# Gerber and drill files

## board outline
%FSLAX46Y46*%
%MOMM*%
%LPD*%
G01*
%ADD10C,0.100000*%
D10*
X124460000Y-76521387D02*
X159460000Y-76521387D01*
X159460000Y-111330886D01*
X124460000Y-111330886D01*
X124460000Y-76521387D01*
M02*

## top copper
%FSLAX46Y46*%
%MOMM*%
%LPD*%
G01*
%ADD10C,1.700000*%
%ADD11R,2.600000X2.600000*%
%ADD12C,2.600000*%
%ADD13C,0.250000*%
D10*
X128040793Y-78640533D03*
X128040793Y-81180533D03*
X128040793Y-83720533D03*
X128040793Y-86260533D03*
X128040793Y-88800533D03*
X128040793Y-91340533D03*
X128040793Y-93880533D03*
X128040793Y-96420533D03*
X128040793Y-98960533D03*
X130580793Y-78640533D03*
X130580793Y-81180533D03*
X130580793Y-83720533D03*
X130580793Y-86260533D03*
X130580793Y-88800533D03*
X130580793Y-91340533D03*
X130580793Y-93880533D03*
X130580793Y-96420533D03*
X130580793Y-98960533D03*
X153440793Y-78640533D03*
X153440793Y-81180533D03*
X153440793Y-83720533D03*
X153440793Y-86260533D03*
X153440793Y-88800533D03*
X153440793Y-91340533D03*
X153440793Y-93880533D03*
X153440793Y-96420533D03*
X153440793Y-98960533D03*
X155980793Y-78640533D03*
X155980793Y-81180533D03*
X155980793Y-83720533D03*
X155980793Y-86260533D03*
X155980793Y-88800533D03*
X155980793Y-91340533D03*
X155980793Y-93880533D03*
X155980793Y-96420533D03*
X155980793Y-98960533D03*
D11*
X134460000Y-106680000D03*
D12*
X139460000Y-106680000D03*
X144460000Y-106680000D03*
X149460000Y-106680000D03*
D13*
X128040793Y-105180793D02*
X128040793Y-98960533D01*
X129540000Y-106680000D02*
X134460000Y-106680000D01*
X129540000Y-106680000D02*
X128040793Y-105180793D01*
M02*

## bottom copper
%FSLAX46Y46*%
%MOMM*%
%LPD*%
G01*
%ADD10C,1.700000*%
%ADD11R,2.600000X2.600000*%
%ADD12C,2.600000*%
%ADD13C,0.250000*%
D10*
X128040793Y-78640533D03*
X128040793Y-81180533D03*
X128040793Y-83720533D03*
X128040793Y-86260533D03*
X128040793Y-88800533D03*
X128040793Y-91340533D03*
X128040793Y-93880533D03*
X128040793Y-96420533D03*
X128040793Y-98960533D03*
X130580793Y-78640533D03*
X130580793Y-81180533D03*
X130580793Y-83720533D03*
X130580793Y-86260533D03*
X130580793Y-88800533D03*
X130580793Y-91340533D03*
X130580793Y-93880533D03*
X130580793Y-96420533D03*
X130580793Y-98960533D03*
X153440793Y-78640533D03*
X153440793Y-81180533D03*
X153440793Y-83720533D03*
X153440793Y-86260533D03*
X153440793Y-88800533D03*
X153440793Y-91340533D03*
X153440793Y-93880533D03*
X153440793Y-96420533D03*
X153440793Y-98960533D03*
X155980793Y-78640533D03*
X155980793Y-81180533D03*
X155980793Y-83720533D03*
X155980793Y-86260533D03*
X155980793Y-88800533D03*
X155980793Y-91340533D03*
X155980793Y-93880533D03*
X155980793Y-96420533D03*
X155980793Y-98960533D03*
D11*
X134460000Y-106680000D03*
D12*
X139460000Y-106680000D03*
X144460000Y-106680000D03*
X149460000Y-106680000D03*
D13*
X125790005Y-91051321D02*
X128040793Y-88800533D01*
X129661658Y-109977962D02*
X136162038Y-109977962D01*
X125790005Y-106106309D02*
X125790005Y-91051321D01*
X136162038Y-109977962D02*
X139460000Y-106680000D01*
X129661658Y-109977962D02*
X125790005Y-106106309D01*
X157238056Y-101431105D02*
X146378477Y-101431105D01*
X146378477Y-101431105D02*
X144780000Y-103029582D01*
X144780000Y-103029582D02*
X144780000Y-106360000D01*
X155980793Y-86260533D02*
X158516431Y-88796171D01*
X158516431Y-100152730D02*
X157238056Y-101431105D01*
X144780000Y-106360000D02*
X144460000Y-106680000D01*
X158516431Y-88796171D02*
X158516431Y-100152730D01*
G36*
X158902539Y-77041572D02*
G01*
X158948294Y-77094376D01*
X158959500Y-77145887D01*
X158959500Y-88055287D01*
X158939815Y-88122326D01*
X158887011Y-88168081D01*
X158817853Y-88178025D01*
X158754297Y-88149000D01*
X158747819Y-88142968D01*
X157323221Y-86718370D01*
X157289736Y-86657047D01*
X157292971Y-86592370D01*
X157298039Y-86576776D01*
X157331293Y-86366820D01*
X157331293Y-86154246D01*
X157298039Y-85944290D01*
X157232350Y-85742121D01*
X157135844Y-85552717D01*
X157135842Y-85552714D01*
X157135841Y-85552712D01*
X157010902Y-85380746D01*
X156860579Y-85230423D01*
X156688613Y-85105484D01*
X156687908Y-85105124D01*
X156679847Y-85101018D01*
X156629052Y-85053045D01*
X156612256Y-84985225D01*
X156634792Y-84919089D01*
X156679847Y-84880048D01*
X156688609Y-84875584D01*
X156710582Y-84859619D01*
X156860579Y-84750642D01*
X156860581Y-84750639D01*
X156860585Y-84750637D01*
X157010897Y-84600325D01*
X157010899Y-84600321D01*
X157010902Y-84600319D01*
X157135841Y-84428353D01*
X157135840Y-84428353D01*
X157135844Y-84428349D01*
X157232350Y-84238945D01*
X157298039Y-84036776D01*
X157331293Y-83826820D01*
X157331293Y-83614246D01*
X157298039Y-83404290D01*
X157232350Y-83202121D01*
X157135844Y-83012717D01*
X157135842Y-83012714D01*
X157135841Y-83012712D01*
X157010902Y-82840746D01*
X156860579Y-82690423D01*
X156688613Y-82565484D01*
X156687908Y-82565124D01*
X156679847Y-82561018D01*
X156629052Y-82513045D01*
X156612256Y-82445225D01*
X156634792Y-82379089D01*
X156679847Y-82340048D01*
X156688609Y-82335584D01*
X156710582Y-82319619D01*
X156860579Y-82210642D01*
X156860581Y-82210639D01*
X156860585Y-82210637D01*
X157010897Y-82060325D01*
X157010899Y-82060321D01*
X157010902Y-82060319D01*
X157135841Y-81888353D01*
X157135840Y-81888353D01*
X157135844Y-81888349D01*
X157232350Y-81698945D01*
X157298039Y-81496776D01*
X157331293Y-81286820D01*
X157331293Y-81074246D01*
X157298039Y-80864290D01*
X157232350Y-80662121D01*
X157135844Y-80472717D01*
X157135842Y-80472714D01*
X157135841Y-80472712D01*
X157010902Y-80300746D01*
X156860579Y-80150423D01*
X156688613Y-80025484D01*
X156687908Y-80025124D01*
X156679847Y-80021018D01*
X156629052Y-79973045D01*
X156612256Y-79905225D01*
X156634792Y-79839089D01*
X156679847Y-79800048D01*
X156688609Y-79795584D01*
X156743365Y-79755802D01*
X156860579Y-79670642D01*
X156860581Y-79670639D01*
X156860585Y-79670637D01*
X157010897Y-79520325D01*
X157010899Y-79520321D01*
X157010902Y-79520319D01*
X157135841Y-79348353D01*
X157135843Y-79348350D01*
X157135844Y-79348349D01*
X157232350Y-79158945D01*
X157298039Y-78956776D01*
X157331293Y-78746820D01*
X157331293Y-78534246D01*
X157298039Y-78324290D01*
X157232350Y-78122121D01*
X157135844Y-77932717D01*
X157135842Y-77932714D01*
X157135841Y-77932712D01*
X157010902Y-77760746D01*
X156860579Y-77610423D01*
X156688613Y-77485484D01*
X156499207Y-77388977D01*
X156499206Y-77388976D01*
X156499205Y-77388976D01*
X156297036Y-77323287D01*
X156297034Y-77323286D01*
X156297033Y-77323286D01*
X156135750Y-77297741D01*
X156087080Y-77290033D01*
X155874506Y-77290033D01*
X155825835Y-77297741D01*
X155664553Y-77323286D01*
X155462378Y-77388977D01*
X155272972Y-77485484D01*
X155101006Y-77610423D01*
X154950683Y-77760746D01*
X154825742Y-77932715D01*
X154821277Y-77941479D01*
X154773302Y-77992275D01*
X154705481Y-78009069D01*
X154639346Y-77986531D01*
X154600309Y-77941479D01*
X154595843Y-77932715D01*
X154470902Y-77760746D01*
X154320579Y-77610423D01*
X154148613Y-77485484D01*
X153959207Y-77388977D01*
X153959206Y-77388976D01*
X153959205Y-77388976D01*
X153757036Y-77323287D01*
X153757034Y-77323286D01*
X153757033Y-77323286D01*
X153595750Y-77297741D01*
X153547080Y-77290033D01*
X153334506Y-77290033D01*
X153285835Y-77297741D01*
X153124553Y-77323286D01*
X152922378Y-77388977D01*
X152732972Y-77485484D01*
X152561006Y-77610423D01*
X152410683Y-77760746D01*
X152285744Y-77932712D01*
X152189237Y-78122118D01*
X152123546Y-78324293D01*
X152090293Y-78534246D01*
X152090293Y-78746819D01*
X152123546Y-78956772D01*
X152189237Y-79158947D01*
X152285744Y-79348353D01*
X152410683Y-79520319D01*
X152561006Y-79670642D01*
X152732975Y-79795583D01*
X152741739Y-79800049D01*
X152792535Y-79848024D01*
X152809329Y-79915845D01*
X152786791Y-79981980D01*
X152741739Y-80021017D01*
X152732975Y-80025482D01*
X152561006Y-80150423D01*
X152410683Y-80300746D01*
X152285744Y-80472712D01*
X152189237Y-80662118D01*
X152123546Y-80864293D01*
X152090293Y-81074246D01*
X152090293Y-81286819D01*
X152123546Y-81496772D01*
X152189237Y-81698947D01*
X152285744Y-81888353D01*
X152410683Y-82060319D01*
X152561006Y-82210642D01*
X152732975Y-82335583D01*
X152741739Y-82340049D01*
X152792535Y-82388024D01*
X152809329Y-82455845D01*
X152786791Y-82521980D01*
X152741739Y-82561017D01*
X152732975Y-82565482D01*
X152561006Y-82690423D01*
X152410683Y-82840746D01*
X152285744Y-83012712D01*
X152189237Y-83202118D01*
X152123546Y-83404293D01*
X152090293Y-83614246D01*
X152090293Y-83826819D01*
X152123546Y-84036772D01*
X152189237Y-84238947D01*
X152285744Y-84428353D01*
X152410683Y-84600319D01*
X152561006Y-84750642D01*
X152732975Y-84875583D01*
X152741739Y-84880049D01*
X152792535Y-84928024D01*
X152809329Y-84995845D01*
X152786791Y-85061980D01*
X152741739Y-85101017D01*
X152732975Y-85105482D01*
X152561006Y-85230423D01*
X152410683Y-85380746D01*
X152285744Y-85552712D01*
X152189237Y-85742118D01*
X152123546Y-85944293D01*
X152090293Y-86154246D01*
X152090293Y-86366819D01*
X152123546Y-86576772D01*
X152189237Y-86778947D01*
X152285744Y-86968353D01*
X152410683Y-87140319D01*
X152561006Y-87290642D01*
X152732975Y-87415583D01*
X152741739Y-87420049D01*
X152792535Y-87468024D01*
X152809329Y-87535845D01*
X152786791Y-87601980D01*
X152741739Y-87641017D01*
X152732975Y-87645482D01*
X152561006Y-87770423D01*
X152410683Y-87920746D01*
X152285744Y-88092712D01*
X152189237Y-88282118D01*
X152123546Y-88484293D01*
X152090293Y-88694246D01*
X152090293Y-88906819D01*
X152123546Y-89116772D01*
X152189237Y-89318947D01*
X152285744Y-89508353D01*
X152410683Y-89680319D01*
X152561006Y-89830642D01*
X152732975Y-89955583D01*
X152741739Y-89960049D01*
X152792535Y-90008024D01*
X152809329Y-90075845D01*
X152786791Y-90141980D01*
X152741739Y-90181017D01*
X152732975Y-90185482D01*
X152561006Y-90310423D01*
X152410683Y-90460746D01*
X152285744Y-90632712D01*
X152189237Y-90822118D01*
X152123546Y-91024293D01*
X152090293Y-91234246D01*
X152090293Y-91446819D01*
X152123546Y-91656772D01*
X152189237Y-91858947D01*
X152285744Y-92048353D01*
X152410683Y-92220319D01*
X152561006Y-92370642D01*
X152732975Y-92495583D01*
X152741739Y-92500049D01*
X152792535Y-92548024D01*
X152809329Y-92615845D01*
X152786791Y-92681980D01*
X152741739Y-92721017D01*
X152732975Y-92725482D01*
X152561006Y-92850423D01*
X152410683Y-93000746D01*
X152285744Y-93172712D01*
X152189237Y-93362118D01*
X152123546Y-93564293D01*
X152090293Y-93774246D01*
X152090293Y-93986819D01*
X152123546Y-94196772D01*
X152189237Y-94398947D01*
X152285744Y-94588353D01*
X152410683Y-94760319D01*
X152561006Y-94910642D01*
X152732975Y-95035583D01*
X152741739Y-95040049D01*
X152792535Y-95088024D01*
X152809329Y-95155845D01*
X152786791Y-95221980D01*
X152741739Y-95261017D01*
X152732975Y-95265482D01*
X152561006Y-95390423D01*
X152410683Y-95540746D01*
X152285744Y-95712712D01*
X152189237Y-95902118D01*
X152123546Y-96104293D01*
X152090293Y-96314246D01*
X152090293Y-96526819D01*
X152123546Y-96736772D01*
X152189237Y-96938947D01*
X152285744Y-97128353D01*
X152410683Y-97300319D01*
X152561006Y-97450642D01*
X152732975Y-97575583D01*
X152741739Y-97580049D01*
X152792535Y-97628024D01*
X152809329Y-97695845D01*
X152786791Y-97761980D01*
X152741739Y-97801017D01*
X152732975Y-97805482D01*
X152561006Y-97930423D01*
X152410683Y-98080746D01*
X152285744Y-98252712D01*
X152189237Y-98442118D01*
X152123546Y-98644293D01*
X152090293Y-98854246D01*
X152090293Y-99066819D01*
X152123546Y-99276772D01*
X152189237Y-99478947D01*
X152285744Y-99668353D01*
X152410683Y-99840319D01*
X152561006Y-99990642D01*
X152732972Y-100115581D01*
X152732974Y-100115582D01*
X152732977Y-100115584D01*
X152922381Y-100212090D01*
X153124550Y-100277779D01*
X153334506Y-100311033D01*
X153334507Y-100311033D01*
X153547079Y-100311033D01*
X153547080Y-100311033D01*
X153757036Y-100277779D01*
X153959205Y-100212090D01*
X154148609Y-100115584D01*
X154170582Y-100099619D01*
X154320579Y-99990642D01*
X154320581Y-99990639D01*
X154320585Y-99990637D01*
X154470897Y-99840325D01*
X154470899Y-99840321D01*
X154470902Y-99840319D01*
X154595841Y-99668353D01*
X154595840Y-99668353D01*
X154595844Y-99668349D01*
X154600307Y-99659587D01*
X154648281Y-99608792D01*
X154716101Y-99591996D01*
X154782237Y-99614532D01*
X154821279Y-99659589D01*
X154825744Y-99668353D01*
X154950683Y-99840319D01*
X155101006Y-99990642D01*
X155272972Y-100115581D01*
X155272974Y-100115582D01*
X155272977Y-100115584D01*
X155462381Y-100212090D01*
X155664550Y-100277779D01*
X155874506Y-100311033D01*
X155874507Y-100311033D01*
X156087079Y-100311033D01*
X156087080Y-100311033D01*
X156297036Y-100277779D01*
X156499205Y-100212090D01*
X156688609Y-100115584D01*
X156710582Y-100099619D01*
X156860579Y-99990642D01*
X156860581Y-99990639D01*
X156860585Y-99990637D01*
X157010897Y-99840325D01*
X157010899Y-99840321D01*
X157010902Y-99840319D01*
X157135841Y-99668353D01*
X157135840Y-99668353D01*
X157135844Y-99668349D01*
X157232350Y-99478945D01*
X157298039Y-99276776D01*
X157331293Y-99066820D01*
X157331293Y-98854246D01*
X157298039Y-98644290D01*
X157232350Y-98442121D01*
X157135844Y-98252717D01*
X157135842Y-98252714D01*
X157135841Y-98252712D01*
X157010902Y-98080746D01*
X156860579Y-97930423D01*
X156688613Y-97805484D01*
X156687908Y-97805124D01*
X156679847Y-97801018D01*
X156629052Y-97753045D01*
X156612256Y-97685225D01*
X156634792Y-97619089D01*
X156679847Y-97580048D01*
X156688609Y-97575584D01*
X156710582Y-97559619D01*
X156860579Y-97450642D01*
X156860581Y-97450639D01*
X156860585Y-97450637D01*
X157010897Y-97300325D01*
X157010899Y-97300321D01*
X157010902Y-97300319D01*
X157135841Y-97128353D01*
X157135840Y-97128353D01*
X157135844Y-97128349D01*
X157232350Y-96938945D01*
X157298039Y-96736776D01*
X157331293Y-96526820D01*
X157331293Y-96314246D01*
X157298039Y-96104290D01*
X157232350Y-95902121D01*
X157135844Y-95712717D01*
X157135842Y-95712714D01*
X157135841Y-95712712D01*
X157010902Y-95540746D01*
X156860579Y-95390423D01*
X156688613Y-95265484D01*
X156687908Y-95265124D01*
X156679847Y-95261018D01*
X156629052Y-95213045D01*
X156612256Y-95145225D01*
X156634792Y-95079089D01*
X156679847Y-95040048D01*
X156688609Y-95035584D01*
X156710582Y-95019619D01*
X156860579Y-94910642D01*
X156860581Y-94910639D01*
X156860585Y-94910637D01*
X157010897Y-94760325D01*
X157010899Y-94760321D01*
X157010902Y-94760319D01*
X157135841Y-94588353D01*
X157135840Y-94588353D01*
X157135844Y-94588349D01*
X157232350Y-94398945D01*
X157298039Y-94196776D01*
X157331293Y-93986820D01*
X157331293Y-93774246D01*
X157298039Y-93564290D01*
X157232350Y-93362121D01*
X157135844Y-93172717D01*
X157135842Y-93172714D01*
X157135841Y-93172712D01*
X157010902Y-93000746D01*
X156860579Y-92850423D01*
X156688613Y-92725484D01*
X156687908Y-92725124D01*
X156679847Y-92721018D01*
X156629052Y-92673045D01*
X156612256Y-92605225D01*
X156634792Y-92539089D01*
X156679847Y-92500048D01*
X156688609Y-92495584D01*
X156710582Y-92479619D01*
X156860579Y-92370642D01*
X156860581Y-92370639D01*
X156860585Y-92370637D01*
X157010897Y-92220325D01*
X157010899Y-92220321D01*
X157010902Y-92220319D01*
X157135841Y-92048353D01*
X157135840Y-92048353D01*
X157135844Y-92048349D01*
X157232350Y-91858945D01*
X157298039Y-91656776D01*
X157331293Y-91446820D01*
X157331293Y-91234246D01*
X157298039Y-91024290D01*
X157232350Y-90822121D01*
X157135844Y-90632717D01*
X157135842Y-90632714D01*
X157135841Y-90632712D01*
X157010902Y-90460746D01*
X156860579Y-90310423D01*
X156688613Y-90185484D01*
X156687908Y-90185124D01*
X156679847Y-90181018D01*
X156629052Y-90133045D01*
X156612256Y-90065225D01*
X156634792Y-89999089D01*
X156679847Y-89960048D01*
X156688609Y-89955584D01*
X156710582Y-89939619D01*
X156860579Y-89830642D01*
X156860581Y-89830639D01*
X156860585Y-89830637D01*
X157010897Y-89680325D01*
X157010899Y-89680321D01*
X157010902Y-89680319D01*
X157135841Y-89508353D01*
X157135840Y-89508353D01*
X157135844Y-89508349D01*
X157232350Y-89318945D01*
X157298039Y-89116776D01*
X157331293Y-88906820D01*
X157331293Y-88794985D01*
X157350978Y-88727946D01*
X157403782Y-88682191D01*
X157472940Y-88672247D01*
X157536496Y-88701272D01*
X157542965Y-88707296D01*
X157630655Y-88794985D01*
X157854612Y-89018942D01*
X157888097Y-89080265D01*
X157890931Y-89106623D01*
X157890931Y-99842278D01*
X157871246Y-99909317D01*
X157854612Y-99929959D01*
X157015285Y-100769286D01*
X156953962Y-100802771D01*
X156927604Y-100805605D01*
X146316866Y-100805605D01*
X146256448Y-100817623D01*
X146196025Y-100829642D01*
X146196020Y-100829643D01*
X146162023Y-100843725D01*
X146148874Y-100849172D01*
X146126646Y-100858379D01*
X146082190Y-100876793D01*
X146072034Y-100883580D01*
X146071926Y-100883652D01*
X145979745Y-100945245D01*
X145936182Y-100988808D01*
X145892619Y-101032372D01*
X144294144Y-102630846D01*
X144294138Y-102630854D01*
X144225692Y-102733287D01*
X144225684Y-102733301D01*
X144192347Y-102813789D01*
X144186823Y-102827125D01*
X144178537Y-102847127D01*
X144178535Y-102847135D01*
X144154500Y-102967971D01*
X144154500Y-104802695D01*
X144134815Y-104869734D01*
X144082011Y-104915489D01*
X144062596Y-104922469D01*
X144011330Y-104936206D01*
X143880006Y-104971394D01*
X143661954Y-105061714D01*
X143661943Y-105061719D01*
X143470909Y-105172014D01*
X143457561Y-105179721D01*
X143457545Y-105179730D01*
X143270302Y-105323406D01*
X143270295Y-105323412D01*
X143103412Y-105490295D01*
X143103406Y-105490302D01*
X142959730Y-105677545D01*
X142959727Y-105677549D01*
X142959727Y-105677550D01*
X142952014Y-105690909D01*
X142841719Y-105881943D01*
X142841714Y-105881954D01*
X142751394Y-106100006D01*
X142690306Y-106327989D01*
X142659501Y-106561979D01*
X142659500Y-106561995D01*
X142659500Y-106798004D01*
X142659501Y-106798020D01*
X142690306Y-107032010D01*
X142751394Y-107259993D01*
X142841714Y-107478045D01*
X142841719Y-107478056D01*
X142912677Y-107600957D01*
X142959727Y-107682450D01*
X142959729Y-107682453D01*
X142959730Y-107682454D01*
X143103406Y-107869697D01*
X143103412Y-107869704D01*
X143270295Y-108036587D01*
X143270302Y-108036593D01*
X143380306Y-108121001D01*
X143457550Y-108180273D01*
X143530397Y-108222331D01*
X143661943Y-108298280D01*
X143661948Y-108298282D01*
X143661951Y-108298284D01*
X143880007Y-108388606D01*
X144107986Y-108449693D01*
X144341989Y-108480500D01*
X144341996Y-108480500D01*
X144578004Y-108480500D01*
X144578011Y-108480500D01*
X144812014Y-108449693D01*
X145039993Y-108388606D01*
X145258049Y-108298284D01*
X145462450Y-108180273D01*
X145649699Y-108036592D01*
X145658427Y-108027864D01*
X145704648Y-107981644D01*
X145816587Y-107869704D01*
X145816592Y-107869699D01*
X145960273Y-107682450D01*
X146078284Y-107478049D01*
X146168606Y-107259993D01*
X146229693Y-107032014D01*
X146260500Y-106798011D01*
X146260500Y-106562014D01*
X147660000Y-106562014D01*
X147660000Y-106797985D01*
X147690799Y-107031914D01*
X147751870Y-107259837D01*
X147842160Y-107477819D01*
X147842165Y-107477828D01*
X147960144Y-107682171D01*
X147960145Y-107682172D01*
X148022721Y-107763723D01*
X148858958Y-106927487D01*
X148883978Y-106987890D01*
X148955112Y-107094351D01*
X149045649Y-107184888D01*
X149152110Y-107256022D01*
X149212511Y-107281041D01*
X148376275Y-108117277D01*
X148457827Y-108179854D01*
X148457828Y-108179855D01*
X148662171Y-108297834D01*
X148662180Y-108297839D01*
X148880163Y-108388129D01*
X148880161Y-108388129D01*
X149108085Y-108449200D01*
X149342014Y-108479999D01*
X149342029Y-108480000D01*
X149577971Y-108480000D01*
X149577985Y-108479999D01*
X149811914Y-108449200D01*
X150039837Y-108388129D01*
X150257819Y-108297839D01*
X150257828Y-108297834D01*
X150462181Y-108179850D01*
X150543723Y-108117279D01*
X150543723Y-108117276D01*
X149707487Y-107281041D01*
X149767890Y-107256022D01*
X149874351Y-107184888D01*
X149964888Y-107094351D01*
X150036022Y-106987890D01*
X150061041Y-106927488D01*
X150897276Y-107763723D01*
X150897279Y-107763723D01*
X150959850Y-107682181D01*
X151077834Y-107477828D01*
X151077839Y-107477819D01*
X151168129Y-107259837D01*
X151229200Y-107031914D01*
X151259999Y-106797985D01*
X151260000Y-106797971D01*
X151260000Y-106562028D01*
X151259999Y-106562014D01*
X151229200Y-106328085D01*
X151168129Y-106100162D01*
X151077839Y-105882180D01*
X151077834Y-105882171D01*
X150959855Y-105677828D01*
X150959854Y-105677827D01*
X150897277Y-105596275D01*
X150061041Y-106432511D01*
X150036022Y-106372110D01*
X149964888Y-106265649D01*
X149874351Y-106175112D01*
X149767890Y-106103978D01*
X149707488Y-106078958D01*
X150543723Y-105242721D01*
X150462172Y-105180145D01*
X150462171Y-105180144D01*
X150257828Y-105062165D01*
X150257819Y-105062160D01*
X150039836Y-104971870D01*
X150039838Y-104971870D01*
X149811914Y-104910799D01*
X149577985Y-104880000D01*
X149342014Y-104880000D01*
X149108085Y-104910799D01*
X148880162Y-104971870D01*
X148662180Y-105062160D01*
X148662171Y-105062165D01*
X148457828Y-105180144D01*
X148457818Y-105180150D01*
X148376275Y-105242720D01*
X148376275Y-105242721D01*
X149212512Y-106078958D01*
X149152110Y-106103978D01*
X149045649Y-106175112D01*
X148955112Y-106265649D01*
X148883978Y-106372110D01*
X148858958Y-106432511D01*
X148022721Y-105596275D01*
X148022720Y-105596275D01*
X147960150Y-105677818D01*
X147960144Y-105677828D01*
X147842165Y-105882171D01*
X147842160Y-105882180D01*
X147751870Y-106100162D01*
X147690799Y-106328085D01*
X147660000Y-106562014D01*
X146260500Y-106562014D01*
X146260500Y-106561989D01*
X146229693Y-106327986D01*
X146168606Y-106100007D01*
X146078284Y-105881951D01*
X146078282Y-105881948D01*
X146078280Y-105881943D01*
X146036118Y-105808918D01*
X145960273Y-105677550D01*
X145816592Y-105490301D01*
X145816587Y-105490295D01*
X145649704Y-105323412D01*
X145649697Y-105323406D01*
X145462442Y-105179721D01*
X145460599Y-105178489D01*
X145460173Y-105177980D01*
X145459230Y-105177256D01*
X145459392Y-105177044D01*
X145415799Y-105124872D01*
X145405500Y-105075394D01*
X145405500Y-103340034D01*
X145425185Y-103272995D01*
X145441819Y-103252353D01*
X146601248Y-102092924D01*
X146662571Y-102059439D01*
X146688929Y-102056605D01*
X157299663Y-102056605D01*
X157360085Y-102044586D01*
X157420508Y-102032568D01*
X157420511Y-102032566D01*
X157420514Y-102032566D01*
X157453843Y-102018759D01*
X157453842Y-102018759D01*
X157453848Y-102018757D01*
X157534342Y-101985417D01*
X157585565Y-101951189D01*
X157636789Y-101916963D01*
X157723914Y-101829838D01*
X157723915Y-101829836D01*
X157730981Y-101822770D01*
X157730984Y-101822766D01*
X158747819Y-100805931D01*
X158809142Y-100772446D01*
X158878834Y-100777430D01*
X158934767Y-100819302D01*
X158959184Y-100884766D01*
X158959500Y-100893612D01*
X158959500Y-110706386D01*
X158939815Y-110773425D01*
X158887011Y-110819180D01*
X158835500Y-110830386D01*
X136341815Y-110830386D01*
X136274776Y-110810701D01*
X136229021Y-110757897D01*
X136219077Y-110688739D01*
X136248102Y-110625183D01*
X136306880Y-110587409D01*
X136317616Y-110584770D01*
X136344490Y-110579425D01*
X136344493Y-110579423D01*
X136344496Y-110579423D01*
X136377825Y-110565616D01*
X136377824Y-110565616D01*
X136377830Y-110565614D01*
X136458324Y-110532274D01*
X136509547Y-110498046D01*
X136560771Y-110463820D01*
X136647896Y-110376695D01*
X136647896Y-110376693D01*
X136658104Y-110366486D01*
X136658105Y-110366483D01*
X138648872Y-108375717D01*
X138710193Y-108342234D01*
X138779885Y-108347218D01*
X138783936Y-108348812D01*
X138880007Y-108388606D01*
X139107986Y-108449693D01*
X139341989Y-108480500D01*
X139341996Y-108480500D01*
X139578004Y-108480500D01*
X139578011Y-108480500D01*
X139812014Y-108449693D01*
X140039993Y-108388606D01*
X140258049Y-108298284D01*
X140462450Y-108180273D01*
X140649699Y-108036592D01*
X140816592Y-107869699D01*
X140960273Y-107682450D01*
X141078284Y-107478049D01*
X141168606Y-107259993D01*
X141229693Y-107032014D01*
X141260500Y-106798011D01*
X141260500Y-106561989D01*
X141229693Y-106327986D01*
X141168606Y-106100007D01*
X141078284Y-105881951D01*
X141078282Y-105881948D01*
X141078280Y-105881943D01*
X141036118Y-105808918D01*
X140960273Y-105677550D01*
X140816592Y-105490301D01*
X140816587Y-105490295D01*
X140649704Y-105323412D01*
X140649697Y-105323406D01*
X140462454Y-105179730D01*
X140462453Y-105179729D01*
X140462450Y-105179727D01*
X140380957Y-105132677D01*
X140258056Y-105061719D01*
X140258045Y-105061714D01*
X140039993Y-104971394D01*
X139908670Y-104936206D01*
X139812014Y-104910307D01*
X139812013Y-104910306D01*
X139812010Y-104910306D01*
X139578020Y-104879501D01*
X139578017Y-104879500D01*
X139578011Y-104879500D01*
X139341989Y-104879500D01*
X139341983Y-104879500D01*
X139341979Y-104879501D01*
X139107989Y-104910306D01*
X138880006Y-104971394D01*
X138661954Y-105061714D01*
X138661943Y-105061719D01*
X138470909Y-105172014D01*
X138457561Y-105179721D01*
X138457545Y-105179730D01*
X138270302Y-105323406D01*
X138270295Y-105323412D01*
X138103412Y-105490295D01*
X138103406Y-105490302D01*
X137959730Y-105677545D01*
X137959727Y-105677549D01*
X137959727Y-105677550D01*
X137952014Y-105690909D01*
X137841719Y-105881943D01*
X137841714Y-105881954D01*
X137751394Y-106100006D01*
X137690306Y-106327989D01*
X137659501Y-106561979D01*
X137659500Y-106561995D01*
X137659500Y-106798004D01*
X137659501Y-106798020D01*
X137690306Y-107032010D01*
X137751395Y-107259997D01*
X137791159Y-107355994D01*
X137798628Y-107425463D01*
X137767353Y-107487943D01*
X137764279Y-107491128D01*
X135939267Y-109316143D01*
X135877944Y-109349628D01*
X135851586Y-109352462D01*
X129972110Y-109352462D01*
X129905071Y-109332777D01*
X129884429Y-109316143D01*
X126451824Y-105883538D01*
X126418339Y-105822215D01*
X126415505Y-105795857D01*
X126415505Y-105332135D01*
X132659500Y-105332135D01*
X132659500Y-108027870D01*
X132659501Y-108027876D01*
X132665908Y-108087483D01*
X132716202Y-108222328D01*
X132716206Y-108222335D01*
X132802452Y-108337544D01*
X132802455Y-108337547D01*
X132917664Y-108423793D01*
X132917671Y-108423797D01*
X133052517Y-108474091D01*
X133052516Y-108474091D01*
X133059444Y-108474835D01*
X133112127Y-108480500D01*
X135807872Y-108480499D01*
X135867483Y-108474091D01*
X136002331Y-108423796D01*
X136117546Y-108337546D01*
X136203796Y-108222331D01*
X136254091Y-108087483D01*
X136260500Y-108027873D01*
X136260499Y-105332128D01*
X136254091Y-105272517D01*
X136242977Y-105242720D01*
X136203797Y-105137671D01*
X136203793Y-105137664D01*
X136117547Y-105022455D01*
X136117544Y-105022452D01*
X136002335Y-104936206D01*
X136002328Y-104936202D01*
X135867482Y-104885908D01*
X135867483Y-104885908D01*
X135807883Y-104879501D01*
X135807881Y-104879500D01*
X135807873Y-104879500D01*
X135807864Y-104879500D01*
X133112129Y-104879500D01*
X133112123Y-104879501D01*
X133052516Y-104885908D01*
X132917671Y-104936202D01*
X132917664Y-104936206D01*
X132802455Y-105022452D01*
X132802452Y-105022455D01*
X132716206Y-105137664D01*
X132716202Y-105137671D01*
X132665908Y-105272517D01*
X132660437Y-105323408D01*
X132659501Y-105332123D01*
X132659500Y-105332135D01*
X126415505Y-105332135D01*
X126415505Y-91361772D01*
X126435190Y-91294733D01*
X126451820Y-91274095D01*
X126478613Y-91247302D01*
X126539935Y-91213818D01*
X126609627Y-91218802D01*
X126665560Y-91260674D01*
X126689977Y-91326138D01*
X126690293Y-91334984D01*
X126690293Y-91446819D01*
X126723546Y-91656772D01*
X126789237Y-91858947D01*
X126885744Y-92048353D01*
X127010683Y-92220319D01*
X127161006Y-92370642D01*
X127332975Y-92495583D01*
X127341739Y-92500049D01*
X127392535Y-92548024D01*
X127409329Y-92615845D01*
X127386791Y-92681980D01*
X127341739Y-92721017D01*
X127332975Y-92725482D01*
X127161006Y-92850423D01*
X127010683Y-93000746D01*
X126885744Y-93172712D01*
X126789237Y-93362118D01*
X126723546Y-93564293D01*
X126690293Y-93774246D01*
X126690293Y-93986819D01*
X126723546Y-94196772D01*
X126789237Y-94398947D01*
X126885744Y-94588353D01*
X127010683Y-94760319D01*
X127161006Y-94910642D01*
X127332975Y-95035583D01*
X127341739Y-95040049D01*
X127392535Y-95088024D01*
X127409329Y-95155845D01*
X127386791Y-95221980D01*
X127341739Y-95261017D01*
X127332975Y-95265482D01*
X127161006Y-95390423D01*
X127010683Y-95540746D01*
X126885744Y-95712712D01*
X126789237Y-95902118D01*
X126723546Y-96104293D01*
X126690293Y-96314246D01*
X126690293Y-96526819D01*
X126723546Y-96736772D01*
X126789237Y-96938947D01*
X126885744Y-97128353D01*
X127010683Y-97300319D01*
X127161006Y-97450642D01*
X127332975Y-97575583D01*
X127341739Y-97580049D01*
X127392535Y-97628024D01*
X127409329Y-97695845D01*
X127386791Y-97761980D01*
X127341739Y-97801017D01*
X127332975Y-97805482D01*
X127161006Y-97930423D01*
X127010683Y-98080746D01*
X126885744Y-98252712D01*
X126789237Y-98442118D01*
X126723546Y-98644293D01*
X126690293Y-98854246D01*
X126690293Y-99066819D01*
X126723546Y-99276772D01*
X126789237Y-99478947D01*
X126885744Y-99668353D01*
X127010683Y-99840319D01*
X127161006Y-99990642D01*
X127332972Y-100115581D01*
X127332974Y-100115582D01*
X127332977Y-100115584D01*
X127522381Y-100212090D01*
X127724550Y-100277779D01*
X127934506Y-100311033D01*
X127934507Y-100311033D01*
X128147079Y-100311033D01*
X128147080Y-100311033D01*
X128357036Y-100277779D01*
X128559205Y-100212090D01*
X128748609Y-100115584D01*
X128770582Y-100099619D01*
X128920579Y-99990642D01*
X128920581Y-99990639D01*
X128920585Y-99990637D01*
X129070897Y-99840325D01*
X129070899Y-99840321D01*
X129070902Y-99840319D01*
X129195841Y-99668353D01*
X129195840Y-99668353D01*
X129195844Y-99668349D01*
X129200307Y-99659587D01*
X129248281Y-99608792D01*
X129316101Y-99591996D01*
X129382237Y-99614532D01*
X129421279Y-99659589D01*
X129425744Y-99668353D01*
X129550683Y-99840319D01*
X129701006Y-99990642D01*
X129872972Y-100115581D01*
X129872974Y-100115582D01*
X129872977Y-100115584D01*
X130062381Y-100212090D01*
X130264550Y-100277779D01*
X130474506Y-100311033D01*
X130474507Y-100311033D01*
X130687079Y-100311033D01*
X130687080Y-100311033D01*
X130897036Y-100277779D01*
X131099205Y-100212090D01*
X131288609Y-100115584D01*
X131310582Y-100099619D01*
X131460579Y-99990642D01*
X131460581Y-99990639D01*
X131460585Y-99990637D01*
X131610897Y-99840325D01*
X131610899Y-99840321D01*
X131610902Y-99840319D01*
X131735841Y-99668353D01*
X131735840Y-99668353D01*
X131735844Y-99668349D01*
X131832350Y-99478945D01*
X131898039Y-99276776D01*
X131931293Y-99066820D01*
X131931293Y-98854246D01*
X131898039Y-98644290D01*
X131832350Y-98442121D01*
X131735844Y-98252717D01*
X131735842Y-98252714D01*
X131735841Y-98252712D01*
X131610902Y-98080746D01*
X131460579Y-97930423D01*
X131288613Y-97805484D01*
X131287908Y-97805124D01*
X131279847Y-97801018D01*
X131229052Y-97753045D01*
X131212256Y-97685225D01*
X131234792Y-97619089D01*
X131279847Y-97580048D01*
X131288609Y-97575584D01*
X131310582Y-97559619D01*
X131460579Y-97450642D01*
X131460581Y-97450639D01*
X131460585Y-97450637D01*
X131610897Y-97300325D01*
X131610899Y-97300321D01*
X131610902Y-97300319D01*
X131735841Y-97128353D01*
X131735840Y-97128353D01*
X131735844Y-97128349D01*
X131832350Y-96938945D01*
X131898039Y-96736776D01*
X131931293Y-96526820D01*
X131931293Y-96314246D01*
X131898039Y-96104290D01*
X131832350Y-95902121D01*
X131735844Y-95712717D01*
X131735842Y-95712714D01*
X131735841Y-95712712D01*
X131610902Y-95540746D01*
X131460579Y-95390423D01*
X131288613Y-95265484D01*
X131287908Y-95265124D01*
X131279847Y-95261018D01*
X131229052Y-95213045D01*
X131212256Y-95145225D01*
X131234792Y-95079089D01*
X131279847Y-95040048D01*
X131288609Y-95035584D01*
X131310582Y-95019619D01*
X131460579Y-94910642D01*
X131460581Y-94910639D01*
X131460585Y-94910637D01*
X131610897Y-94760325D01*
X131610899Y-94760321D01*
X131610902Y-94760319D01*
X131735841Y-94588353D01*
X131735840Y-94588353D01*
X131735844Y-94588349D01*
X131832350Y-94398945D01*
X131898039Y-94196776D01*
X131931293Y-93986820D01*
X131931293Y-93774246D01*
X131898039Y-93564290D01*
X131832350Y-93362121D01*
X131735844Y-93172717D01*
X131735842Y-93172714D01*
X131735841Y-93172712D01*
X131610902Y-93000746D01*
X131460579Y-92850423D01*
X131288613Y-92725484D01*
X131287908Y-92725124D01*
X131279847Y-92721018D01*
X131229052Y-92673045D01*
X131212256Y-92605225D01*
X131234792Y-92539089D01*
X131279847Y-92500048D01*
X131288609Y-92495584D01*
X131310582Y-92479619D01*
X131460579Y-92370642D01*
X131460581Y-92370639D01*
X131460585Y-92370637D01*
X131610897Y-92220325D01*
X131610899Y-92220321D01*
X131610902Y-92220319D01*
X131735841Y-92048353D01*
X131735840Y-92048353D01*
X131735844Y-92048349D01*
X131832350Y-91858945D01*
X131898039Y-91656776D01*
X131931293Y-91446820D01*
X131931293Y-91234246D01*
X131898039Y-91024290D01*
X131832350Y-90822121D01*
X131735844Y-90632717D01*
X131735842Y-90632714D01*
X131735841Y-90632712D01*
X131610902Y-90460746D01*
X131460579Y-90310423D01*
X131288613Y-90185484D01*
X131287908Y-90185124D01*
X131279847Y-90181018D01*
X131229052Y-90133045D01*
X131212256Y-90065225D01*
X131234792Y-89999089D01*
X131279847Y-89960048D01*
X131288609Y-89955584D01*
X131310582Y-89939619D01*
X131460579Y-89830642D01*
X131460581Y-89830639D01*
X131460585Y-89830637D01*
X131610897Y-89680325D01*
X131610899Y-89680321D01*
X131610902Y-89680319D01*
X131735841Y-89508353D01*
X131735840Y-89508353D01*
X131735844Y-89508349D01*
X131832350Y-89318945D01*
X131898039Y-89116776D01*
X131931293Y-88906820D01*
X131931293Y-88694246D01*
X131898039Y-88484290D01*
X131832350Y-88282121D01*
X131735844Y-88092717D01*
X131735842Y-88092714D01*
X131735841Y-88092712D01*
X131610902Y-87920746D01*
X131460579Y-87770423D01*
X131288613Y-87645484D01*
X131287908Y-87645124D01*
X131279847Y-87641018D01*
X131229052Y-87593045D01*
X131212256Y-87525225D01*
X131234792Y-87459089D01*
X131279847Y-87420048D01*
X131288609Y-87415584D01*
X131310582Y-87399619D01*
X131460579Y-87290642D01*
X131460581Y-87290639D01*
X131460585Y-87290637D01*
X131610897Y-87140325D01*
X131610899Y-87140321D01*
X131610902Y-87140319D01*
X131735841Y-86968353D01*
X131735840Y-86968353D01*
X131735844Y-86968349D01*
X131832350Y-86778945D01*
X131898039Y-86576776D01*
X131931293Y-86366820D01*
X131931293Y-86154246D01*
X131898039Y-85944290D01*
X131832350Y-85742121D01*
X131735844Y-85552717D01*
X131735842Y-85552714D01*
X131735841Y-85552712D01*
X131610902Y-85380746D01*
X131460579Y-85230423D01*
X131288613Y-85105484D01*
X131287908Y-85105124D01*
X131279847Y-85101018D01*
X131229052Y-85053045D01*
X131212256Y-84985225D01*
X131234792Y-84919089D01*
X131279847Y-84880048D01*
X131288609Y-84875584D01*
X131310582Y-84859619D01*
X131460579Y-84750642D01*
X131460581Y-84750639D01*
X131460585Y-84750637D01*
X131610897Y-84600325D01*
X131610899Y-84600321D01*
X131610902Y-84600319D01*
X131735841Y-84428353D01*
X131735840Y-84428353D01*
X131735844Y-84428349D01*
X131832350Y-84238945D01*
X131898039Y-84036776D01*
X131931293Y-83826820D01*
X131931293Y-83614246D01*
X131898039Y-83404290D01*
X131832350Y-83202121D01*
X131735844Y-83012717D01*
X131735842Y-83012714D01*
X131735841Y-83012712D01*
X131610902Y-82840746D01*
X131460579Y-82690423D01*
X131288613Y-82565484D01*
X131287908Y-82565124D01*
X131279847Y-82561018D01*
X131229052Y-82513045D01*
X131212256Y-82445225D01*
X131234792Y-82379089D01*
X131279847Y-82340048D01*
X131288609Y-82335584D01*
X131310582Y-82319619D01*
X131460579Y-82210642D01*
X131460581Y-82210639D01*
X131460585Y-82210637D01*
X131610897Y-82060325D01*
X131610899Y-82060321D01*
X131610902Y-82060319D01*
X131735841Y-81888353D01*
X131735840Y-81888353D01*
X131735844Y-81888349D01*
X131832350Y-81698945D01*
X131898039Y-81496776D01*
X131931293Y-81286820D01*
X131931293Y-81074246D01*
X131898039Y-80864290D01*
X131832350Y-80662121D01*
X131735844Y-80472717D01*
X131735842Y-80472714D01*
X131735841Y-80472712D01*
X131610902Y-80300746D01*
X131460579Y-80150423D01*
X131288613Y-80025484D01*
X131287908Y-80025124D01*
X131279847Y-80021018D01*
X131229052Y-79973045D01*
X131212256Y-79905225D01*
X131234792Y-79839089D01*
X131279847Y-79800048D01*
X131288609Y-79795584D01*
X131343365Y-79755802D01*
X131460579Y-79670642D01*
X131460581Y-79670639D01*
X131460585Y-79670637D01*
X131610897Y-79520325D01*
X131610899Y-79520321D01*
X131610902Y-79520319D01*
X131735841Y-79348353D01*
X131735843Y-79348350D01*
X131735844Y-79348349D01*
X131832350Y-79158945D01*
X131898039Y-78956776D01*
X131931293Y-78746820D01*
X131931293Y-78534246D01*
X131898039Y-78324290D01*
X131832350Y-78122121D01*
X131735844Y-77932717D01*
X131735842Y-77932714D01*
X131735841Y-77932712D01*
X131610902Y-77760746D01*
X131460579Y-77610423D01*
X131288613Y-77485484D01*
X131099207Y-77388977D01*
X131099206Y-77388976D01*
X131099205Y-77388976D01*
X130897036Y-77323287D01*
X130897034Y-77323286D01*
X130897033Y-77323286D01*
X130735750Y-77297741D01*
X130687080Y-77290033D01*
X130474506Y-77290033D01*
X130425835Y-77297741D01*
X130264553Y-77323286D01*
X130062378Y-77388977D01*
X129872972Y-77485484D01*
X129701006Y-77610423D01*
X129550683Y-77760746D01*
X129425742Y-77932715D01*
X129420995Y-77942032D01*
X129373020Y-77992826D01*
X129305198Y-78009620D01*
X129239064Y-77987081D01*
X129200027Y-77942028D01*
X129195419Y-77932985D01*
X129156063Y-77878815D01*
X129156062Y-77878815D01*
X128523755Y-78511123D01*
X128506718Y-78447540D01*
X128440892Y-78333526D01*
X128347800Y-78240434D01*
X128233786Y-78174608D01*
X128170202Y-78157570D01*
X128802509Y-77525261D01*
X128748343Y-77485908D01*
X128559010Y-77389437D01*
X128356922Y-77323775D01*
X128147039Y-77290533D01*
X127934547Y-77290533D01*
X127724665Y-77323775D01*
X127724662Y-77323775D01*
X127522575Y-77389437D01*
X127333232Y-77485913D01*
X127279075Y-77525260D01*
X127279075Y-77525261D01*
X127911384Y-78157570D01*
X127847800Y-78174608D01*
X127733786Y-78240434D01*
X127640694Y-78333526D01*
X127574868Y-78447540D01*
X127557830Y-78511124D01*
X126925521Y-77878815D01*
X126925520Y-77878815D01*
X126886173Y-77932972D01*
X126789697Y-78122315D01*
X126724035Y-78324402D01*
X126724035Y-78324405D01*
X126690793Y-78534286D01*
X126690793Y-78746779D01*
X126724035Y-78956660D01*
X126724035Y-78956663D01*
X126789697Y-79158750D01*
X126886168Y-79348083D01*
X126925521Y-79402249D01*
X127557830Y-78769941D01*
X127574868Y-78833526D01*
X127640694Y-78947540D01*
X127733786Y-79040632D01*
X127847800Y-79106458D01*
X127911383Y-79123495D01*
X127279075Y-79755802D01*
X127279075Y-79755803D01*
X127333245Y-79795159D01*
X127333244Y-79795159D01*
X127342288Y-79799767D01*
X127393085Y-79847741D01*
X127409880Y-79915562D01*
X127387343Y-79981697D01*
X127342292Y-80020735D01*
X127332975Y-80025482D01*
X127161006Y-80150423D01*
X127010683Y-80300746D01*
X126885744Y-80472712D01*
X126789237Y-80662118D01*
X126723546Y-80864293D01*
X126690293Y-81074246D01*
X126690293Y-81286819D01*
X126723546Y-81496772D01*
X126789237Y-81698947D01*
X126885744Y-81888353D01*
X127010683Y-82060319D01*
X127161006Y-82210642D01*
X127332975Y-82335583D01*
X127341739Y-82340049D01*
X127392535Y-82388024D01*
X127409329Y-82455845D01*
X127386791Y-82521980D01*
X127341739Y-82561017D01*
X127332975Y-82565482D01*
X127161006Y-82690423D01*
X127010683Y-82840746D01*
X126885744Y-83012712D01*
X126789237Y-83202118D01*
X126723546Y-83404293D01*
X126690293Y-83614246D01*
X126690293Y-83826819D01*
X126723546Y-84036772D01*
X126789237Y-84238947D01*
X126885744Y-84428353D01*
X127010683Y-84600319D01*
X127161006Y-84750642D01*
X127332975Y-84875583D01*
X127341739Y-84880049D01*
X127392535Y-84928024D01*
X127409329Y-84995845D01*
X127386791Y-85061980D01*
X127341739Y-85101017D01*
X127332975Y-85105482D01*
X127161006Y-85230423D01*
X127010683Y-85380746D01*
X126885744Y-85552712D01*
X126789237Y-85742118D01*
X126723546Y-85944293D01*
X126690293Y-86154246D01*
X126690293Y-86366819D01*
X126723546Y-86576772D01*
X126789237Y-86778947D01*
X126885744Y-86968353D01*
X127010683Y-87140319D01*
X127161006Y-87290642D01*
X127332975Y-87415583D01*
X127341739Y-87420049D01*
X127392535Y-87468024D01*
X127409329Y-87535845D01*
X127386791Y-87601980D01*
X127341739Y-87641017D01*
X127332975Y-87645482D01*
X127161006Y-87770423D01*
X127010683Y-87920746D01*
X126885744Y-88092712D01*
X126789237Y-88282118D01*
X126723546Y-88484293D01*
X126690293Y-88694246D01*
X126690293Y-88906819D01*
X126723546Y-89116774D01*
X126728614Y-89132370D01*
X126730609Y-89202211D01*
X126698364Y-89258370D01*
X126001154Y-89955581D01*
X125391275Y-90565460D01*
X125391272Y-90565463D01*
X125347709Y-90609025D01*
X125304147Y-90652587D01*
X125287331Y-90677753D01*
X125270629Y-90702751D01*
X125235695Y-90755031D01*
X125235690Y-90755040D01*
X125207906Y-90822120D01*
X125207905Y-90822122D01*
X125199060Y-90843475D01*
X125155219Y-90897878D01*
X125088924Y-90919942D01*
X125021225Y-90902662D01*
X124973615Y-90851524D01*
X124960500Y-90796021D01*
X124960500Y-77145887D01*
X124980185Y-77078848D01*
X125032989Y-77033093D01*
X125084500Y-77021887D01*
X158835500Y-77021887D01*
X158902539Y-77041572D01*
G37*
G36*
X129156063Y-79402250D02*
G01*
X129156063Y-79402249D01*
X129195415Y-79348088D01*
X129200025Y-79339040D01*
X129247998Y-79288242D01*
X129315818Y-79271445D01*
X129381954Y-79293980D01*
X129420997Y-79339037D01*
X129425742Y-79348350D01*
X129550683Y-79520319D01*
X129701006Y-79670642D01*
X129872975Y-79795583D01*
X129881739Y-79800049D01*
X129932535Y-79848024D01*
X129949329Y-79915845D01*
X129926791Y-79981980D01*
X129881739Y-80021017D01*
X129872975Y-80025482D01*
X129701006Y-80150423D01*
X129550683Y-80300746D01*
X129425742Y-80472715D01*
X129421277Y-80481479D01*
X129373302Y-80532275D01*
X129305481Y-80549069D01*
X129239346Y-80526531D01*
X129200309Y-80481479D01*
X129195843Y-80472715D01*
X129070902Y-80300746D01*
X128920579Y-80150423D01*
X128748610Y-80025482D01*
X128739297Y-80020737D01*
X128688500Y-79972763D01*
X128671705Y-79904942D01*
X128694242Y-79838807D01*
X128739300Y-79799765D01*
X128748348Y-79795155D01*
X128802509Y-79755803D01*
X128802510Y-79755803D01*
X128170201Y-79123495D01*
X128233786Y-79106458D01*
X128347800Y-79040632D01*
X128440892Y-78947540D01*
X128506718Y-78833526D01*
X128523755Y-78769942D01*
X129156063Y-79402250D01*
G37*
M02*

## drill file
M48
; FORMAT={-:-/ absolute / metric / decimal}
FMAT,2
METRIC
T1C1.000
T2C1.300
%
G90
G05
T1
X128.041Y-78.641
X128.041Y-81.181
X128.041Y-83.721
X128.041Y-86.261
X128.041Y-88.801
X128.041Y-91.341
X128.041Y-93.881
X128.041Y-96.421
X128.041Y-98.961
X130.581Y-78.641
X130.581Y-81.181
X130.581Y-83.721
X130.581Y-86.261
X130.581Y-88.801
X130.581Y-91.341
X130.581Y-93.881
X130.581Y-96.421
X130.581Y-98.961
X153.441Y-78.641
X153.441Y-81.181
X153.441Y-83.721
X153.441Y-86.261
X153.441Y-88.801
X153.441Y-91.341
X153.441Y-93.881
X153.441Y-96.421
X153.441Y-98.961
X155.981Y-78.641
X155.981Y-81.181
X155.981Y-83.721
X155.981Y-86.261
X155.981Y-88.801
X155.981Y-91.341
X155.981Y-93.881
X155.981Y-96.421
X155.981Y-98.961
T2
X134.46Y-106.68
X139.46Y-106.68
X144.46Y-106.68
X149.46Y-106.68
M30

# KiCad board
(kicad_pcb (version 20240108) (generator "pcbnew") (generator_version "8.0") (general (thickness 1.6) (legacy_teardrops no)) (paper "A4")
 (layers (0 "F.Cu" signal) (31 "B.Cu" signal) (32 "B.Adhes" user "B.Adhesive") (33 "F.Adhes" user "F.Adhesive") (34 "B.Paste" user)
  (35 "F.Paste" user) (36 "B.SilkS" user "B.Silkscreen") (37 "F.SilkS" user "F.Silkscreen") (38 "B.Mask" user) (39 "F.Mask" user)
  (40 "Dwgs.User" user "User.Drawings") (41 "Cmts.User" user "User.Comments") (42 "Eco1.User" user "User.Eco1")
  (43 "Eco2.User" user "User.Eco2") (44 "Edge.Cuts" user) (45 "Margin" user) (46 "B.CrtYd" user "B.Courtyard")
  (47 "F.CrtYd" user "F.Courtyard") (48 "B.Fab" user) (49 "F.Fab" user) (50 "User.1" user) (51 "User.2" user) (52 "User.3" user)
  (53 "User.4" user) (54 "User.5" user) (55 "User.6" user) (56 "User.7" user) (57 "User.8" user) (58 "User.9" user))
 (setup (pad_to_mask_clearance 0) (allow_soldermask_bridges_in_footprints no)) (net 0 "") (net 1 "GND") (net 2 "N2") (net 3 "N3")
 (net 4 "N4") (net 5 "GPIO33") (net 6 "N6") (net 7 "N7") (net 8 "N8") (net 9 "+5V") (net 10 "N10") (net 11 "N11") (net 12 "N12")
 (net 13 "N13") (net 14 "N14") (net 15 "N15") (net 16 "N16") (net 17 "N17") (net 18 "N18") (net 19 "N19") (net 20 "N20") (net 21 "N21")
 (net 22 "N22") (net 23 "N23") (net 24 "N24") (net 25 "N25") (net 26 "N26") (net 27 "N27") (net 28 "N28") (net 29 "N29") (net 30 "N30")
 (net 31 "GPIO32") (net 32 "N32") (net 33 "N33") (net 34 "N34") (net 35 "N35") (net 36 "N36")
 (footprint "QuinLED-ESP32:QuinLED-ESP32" (layer "F.Cu") (at 142.112393 93.220133)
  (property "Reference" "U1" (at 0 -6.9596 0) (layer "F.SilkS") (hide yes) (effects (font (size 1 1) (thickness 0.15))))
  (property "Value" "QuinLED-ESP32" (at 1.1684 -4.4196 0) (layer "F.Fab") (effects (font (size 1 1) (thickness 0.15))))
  (pad "1" thru_hole circle (at -14.0716 -14.5796) (size 1.7 1.7) (drill 1) (layers "*.Cu" "*.Mask") (remove_unused_layers no) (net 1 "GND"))
  (pad "2" thru_hole circle (at -14.0716 -12.0396) (size 1.7 1.7) (drill 1) (layers "*.Cu" "*.Mask") (remove_unused_layers no) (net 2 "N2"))
  (pad "3" thru_hole circle (at -14.0716 -9.4996) (size 1.7 1.7) (drill 1) (layers "*.Cu" "*.Mask") (remove_unused_layers no) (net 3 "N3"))
  (pad "4" thru_hole circle (at -14.0716 -6.9596) (size 1.7 1.7) (drill 1) (layers "*.Cu" "*.Mask") (remove_unused_layers no) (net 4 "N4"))
  (pad "5" thru_hole circle (at -14.0716 -4.4196) (size 1.7 1.7) (drill 1) (layers "*.Cu" "*.Mask") (remove_unused_layers no)
   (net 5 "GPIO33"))
  (pad "6" thru_hole circle (at -14.0716 -1.8796) (size 1.7 1.7) (drill 1) (layers "*.Cu" "*.Mask") (remove_unused_layers no) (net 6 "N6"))
  (pad "7" thru_hole circle (at -14.0716 0.6604) (size 1.7 1.7) (drill 1) (layers "*.Cu" "*.Mask") (remove_unused_layers no) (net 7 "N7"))
  (pad "8" thru_hole circle (at -14.0716 3.2004) (size 1.7 1.7) (drill 1) (layers "*.Cu" "*.Mask") (remove_unused_layers no) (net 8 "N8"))
  (pad "9" thru_hole circle (at -14.0716 5.7404) (size 1.7 1.7) (drill 1) (layers "*.Cu" "*.Mask") (remove_unused_layers no) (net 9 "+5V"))
  (pad "10" thru_hole circle (at -11.5316 -14.5796) (size 1.7 1.7) (drill 1) (layers "*.Cu" "*.Mask") (remove_unused_layers no)
   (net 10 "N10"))
  (pad "11" thru_hole circle (at -11.5316 -12.0396) (size 1.7 1.7) (drill 1) (layers "*.Cu" "*.Mask") (remove_unused_layers no)
   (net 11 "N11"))
  (pad "12" thru_hole circle (at -11.5316 -9.4996) (size 1.7 1.7) (drill 1) (layers "*.Cu" "*.Mask") (remove_unused_layers no)
   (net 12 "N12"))
  (pad "13" thru_hole circle (at -11.5316 -6.9596) (size 1.7 1.7) (drill 1) (layers "*.Cu" "*.Mask") (remove_unused_layers no)
   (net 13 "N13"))
  (pad "14" thru_hole circle (at -11.5316 -4.4196) (size 1.7 1.7) (drill 1) (layers "*.Cu" "*.Mask") (remove_unused_layers no)
   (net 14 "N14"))
  (pad "15" thru_hole circle (at -11.5316 -1.8796) (size 1.7 1.7) (drill 1) (layers "*.Cu" "*.Mask") (remove_unused_layers no)
   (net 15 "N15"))
  (pad "16" thru_hole circle (at -11.5316 0.6604) (size 1.7 1.7) (drill 1) (layers "*.Cu" "*.Mask") (remove_unused_layers no) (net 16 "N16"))
  (pad "17" thru_hole circle (at -11.5316 3.2004) (size 1.7 1.7) (drill 1) (layers "*.Cu" "*.Mask") (remove_unused_layers no) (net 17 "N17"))
  (pad "18" thru_hole circle (at -11.5316 5.7404) (size 1.7 1.7) (drill 1) (layers "*.Cu" "*.Mask") (remove_unused_layers no) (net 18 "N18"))
  (pad "19" thru_hole circle (at 11.3284 -14.5796) (size 1.7 1.7) (drill 1) (layers "*.Cu" "*.Mask") (remove_unused_layers no)
   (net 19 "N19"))
  (pad "20" thru_hole circle (at 11.3284 -12.0396) (size 1.7 1.7) (drill 1) (layers "*.Cu" "*.Mask") (remove_unused_layers no)
   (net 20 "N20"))
  (pad "21" thru_hole circle (at 11.3284 -9.4996) (size 1.7 1.7) (drill 1) (layers "*.Cu" "*.Mask") (remove_unused_layers no) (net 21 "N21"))
  (pad "22" thru_hole circle (at 11.3284 -6.9596) (size 1.7 1.7) (drill 1) (layers "*.Cu" "*.Mask") (remove_unused_layers no) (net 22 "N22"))
  (pad "23" thru_hole circle (at 11.3284 -4.4196) (size 1.7 1.7) (drill 1) (layers "*.Cu" "*.Mask") (remove_unused_layers no) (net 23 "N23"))
  (pad "24" thru_hole circle (at 11.3284 -1.8796) (size 1.7 1.7) (drill 1) (layers "*.Cu" "*.Mask") (remove_unused_layers no) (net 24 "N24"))
  (pad "25" thru_hole circle (at 11.3284 0.6604) (size 1.7 1.7) (drill 1) (layers "*.Cu" "*.Mask") (remove_unused_layers no) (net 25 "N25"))
  (pad "26" thru_hole circle (at 11.3284 3.2004) (size 1.7 1.7) (drill 1) (layers "*.Cu" "*.Mask") (remove_unused_layers no) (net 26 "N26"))
  (pad "27" thru_hole circle (at 11.3284 5.7404) (size 1.7 1.7) (drill 1) (layers "*.Cu" "*.Mask") (remove_unused_layers no) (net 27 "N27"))
  (pad "28" thru_hole circle (at 13.8684 -14.5796) (size 1.7 1.7) (drill 1) (layers "*.Cu" "*.Mask") (remove_unused_layers no)
   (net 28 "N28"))
  (pad "29" thru_hole circle (at 13.8684 -12.0396) (size 1.7 1.7) (drill 1) (layers "*.Cu" "*.Mask") (remove_unused_layers no)
   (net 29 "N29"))
  (pad "30" thru_hole circle (at 13.8684 -9.4996) (size 1.7 1.7) (drill 1) (layers "*.Cu" "*.Mask") (remove_unused_layers no) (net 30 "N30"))
  (pad "31" thru_hole circle (at 13.8684 -6.9596) (size 1.7 1.7) (drill 1) (layers "*.Cu" "*.Mask") (remove_unused_layers no)
   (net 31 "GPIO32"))
  (pad "32" thru_hole circle (at 13.8684 -4.4196) (size 1.7 1.7) (drill 1) (layers "*.Cu" "*.Mask") (remove_unused_layers no) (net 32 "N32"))
  (pad "33" thru_hole circle (at 13.8684 -1.8796) (size 1.7 1.7) (drill 1) (layers "*.Cu" "*.Mask") (remove_unused_layers no) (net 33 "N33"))
  (pad "34" thru_hole circle (at 13.8684 0.6604) (size 1.7 1.7) (drill 1) (layers "*.Cu" "*.Mask") (remove_unused_layers no) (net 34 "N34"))
  (pad "35" thru_hole circle (at 13.8684 3.2004) (size 1.7 1.7) (drill 1) (layers "*.Cu" "*.Mask") (remove_unused_layers no) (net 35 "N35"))
  (pad "36" thru_hole circle (at 13.8684 5.7404) (size 1.7 1.7) (drill 1) (layers "*.Cu" "*.Mask") (remove_unused_layers no) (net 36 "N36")))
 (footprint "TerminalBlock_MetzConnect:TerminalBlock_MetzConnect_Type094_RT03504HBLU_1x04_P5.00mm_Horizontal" (layer "F.Cu")
  (at 134.46 106.68)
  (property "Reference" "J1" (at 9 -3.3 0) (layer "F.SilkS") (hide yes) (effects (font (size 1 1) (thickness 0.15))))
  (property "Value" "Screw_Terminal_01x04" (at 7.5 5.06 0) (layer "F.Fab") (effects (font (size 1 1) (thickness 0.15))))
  (pad "1" thru_hole rect (at 0 0) (size 2.6 2.6) (drill 1.3) (layers "*.Cu" "*.Mask") (remove_unused_layers no) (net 9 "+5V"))
  (pad "2" thru_hole circle (at 5 0) (size 2.6 2.6) (drill 1.3) (layers "*.Cu" "*.Mask") (remove_unused_layers no) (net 5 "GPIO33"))
  (pad "3" thru_hole circle (at 10 0) (size 2.6 2.6) (drill 1.3) (layers "*.Cu" "*.Mask") (remove_unused_layers no) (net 31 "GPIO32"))
  (pad "4" thru_hole circle (at 15 0) (size 2.6 2.6) (drill 1.3) (layers "*.Cu" "*.Mask") (remove_unused_layers no) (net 1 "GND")))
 (gr_rect (start 124.46 76.521387) (end 159.46 111.330886) (stroke (width 0.1) (type default)) (fill none) (layer "Edge.Cuts"))
 (segment (start 125.790005 91.051321) (end 128.040793 88.800533) (width 0.25) (layer "B.Cu") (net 5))
 (segment (start 129.661658 109.977962) (end 136.162038 109.977962) (width 0.25) (layer "B.Cu") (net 5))
 (segment (start 125.790005 106.106309) (end 125.790005 91.051321) (width 0.25) (layer "B.Cu") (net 5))
 (segment (start 136.162038 109.977962) (end 139.46 106.68) (width 0.25) (layer "B.Cu") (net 5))
 (segment (start 129.661658 109.977962) (end 125.790005 106.106309) (width 0.25) (layer "B.Cu") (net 5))
 (segment (start 157.238056 101.431105) (end 146.378477 101.431105) (width 0.25) (layer "B.Cu") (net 31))
 (segment (start 146.378477 101.431105) (end 144.78 103.029582) (width 0.25) (layer "B.Cu") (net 31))
 (segment (start 144.78 103.029582) (end 144.78 106.36) (width 0.25) (layer "B.Cu") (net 31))
 (segment (start 155.980793 86.260533) (end 158.516431 88.796171) (width 0.25) (layer "B.Cu") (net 31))
 (segment (start 158.516431 100.15273) (end 157.238056 101.431105) (width 0.25) (layer "B.Cu") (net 31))
 (segment (start 144.78 106.36) (end 144.46 106.68) (width 0.25) (layer "B.Cu") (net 31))
 (segment (start 158.516431 88.796171) (end 158.516431 100.15273) (width 0.25) (layer "B.Cu") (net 31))
 (segment (start 128.040793 105.180793) (end 128.040793 98.960533) (width 0.25) (layer "F.Cu") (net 9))
 (segment (start 129.54 106.68) (end 134.46 106.68) (width 0.25) (layer "F.Cu") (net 9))
 (segment (start 129.54 106.68) (end 128.040793 105.180793) (width 0.25) (layer "F.Cu") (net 9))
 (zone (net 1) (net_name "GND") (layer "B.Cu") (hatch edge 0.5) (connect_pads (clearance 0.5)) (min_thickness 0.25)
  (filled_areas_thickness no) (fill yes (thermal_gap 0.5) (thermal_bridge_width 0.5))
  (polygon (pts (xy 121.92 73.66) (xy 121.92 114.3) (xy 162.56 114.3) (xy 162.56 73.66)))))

